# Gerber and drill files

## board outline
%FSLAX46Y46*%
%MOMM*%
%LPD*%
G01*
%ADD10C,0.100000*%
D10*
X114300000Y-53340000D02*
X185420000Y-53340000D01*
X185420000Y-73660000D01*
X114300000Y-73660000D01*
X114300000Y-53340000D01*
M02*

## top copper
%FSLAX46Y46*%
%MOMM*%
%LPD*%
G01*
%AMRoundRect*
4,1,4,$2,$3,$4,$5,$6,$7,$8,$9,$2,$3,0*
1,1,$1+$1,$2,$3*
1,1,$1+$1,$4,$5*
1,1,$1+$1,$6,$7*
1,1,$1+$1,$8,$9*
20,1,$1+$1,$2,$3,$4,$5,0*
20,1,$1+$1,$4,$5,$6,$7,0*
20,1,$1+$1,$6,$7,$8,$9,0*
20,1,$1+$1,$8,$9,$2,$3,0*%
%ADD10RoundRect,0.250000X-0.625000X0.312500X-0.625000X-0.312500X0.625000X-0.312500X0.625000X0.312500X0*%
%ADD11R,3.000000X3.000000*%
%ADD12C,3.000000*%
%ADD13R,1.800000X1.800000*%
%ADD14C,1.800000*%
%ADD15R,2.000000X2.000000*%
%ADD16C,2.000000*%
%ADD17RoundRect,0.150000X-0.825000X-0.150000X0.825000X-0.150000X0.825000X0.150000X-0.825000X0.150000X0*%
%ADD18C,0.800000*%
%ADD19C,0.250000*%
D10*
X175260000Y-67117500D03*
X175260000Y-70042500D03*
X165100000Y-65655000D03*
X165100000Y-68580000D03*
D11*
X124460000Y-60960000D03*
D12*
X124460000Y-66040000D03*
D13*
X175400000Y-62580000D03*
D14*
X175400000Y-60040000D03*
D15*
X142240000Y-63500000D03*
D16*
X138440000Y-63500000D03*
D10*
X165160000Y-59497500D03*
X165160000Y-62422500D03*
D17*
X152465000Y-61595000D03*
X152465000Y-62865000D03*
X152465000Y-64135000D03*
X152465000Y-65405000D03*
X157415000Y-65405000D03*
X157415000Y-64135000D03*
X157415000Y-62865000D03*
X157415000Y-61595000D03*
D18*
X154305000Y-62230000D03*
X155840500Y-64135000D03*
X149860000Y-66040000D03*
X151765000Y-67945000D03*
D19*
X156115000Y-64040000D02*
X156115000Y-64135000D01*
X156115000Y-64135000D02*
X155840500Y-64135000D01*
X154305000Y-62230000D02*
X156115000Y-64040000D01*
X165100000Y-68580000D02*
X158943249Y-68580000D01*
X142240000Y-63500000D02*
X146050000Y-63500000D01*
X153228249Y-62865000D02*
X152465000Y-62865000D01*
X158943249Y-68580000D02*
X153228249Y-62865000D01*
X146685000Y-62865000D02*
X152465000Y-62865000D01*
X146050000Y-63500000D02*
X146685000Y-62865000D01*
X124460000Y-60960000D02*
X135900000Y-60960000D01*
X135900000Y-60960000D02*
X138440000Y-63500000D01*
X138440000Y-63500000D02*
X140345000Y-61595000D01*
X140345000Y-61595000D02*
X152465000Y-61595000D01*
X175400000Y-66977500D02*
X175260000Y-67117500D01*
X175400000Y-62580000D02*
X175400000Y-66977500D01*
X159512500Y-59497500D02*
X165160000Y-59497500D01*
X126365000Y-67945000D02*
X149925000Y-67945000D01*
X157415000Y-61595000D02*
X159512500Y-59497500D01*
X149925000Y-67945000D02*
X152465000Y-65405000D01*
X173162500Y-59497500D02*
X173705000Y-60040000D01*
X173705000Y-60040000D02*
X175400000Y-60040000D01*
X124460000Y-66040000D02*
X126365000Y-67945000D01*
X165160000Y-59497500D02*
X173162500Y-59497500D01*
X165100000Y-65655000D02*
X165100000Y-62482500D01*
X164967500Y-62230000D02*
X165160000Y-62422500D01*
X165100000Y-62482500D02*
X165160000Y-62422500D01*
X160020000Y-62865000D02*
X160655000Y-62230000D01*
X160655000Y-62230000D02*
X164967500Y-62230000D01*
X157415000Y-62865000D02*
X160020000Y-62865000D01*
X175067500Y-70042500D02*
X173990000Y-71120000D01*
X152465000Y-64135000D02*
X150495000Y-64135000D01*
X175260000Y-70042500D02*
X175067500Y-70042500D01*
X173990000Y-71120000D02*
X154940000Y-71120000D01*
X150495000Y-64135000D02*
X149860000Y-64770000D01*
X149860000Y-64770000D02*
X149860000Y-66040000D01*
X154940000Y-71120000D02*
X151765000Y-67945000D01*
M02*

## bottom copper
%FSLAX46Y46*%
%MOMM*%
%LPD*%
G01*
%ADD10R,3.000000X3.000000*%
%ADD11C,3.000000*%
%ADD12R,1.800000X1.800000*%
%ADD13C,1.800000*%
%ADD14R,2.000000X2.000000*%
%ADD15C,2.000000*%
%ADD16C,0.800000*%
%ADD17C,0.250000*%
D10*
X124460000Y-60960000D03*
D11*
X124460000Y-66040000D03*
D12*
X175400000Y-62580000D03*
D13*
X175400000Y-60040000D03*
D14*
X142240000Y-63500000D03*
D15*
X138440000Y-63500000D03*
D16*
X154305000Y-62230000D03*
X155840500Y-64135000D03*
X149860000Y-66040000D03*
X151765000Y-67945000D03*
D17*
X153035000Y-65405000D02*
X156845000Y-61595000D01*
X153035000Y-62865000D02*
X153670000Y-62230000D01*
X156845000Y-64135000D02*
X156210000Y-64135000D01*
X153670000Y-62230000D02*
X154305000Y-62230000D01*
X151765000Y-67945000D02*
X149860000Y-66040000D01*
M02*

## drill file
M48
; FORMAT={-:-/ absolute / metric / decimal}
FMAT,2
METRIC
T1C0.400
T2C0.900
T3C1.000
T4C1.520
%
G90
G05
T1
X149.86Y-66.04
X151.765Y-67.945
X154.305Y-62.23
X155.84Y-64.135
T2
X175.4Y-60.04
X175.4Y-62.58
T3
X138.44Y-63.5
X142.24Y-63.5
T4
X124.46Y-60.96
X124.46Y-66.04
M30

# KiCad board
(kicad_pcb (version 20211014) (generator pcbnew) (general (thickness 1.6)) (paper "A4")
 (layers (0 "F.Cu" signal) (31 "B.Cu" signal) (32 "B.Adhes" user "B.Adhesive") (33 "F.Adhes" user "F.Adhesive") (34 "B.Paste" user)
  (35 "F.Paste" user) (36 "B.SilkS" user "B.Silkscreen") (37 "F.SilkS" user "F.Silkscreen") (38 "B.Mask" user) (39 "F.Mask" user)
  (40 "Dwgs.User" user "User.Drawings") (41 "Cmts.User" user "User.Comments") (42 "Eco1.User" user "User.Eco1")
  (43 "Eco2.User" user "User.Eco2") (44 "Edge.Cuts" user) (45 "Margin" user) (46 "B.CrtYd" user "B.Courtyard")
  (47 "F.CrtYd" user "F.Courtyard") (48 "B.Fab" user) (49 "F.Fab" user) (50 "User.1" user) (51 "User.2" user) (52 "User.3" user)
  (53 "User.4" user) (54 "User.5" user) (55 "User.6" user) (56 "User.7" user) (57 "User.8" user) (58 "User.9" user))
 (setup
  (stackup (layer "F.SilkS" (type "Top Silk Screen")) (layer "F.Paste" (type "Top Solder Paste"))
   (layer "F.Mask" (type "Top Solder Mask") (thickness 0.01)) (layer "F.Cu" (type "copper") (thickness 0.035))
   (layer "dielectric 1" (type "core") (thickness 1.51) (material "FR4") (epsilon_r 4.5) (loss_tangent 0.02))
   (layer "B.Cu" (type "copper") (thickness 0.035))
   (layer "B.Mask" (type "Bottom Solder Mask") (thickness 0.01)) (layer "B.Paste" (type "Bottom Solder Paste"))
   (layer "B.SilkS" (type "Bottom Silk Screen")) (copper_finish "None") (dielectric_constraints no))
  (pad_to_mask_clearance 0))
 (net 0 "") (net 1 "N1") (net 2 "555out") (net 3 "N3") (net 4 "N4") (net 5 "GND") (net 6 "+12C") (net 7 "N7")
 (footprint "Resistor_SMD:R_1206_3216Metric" (layer "F.Cu") (at 175.26 68.58 -90)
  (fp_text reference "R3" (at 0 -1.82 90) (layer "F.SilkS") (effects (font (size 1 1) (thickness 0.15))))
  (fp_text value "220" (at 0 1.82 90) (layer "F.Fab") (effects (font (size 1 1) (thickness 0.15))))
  (pad "1" smd roundrect (at -1.4625 0 270) (size 1.125 1.75) (layers "F.Cu" "F.Paste" "F.Mask") (roundrect_rratio 0.222222) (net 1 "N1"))
  (pad "2" smd roundrect (at 1.4625 0 270) (size 1.125 1.75) (layers "F.Cu" "F.Paste" "F.Mask") (roundrect_rratio 0.222222) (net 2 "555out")))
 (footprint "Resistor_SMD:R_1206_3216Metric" (layer "F.Cu") (at 165.1 67.1175 -90)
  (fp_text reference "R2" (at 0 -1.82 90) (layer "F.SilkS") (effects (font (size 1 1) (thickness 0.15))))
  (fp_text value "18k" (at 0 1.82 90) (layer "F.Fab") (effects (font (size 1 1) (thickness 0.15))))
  (pad "1" smd roundrect (at -1.4625 0 270) (size 1.125 1.75) (layers "F.Cu" "F.Paste" "F.Mask") (roundrect_rratio 0.222222) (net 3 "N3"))
  (pad "2" smd roundrect (at 1.4625 0 270) (size 1.125 1.75) (layers "F.Cu" "F.Paste" "F.Mask") (roundrect_rratio 0.222222) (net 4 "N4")))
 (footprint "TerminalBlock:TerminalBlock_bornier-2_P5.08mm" (layer "F.Cu") (at 124.46 60.96 -90)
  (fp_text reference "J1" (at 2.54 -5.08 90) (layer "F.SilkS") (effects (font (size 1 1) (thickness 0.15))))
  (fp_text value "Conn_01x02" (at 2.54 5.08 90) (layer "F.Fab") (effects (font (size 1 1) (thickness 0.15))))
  (pad "1" thru_hole rect (at 0 0 270) (size 3 3) (drill 1.52) (layers *.Cu *.Mask) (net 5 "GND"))
  (pad "2" thru_hole circle (at 5.08 0 270) (size 3 3) (drill 1.52) (layers *.Cu *.Mask) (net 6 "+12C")))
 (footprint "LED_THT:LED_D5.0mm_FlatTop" (layer "F.Cu") (at 175.4 62.58 90)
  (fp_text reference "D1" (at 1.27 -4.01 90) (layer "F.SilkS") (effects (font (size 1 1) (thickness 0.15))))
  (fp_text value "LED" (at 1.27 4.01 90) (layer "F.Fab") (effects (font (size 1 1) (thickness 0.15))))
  (pad "1" thru_hole rect (at 0 0 90) (size 1.8 1.8) (drill 0.9) (layers *.Cu *.Mask) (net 1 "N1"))
  (pad "2" thru_hole circle (at 2.54 0 90) (size 1.8 1.8) (drill 0.9) (layers *.Cu *.Mask) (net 6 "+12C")))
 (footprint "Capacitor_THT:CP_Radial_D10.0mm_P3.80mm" (layer "F.Cu") (at 142.24 63.5 180)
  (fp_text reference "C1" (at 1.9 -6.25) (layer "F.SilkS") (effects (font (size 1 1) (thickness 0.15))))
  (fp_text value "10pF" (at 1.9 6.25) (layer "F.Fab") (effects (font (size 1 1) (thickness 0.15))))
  (pad "1" thru_hole rect (at 0 0 180) (size 2 2) (drill 1) (layers *.Cu *.Mask) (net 4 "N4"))
  (pad "2" thru_hole circle (at 3.8 0 180) (size 2 2) (drill 1) (layers *.Cu *.Mask) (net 5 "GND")))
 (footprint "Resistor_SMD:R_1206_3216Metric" (layer "F.Cu") (at 165.16 60.96 -90)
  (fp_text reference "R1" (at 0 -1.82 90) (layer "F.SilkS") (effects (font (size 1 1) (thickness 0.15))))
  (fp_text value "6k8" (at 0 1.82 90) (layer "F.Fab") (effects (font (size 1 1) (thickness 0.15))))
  (pad "1" smd roundrect (at -1.4625 0 270) (size 1.125 1.75) (layers "F.Cu" "F.Paste" "F.Mask") (roundrect_rratio 0.222222) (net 6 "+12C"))
  (pad "2" smd roundrect (at 1.4625 0 270) (size 1.125 1.75) (layers "F.Cu" "F.Paste" "F.Mask") (roundrect_rratio 0.222222) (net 3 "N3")))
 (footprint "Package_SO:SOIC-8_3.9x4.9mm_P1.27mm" (layer "F.Cu") (at 154.94 63.5)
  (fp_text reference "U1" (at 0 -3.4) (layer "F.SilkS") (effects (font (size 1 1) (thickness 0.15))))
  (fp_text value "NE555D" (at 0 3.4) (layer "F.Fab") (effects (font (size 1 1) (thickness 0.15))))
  (pad "1" smd roundrect (at -2.475 -1.905) (size 1.95 0.6) (layers "F.Cu" "F.Paste" "F.Mask") (roundrect_rratio 0.25) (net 5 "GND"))
  (pad "2" smd roundrect (at -2.475 -0.635) (size 1.95 0.6) (layers "F.Cu" "F.Paste" "F.Mask") (roundrect_rratio 0.25) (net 4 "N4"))
  (pad "3" smd roundrect (at -2.475 0.635) (size 1.95 0.6) (layers "F.Cu" "F.Paste" "F.Mask") (roundrect_rratio 0.25) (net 2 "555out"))
  (pad "4" smd roundrect (at -2.475 1.905) (size 1.95 0.6) (layers "F.Cu" "F.Paste" "F.Mask") (roundrect_rratio 0.25) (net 6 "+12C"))
  (pad "5" smd roundrect (at 2.475 1.905) (size 1.95 0.6) (layers "F.Cu" "F.Paste" "F.Mask") (roundrect_rratio 0.25) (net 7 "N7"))
  (pad "6" smd roundrect (at 2.475 0.635) (size 1.95 0.6) (layers "F.Cu" "F.Paste" "F.Mask") (roundrect_rratio 0.25) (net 4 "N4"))
  (pad "7" smd roundrect (at 2.475 -0.635) (size 1.95 0.6) (layers "F.Cu" "F.Paste" "F.Mask") (roundrect_rratio 0.25) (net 3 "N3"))
  (pad "8" smd roundrect (at 2.475 -1.905) (size 1.95 0.6) (layers "F.Cu" "F.Paste" "F.Mask") (roundrect_rratio 0.25) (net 6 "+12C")))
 (gr_rect (start 114.3 53.34) (end 185.42 73.66) (layer "Edge.Cuts") (width 0.1) (fill none))
 (segment (start 156.115 64.04) (end 156.115 64.135) (width 0.25) (layer "F.Cu") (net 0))
 (segment (start 156.115 64.135) (end 155.8405 64.135) (width 0.25) (layer "F.Cu") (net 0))
 (segment (start 154.305 62.23) (end 156.115 64.04) (width 0.25) (layer "F.Cu") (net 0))
 (via (at 154.305 62.23) (size 0.8) (drill 0.4) (layers "F.Cu" "B.Cu") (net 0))
 (via (at 155.8405 64.135) (size 0.8) (drill 0.4) (layers "F.Cu" "B.Cu") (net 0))
 (segment (start 153.035 65.405) (end 156.845 61.595) (width 0.25) (layer "B.Cu") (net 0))
 (segment (start 153.035 62.865) (end 153.67 62.23) (width 0.25) (layer "B.Cu") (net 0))
 (segment (start 156.845 64.135) (end 156.21 64.135) (width 0.25) (layer "B.Cu") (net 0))
 (segment (start 153.67 62.23) (end 154.305 62.23) (width 0.25) (layer "B.Cu") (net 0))
 (segment (start 165.1 68.58) (end 158.943249 68.58) (width 0.25) (layer "F.Cu") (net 4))
 (segment (start 142.24 63.5) (end 146.05 63.5) (width 0.25) (layer "F.Cu") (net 4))
 (segment (start 153.228249 62.865) (end 152.465 62.865) (width 0.25) (layer "F.Cu") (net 4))
 (segment (start 158.943249 68.58) (end 153.228249 62.865) (width 0.25) (layer "F.Cu") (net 4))
 (segment (start 146.685 62.865) (end 152.465 62.865) (width 0.25) (layer "F.Cu") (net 4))
 (segment (start 146.05 63.5) (end 146.685 62.865) (width 0.25) (layer "F.Cu") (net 4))
 (segment (start 124.46 60.96) (end 135.9 60.96) (width 0.25) (layer "F.Cu") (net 5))
 (segment (start 135.9 60.96) (end 138.44 63.5) (width 0.25) (layer "F.Cu") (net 5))
 (segment (start 138.44 63.5) (end 140.345 61.595) (width 0.25) (layer "F.Cu") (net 5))
 (segment (start 140.345 61.595) (end 152.465 61.595) (width 0.25) (layer "F.Cu") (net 5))
 (segment (start 175.4 66.9775) (end 175.26 67.1175) (width 0.25) (layer "F.Cu") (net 1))
 (segment (start 175.4 62.58) (end 175.4 66.9775) (width 0.25) (layer "F.Cu") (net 1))
 (segment (start 159.5125 59.4975) (end 165.16 59.4975) (width 0.25) (layer "F.Cu") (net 6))
 (segment (start 126.365 67.945) (end 149.925 67.945) (width 0.25) (layer "F.Cu") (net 6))
 (segment (start 157.415 61.595) (end 159.5125 59.4975) (width 0.25) (layer "F.Cu") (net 6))
 (segment (start 149.925 67.945) (end 152.465 65.405) (width 0.25) (layer "F.Cu") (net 6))
 (segment (start 173.1625 59.4975) (end 173.705 60.04) (width 0.25) (layer "F.Cu") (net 6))
 (segment (start 173.705 60.04) (end 175.4 60.04) (width 0.25) (layer "F.Cu") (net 6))
 (segment (start 124.46 66.04) (end 126.365 67.945) (width 0.25) (layer "F.Cu") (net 6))
 (segment (start 165.16 59.4975) (end 173.1625 59.4975) (width 0.25) (layer "F.Cu") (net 6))
 (segment (start 165.1 65.655) (end 165.1 62.4825) (width 0.25) (layer "F.Cu") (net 3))
 (segment (start 164.9675 62.23) (end 165.16 62.4225) (width 0.25) (layer "F.Cu") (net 3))
 (segment (start 165.1 62.4825) (end 165.16 62.4225) (width 0.25) (layer "F.Cu") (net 3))
 (segment (start 160.02 62.865) (end 160.655 62.23) (width 0.25) (layer "F.Cu") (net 3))
 (segment (start 160.655 62.23) (end 164.9675 62.23) (width 0.25) (layer "F.Cu") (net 3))
 (segment (start 157.415 62.865) (end 160.02 62.865) (width 0.25) (layer "F.Cu") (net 3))
 (segment (start 175.0675 70.0425) (end 173.99 71.12) (width 0.25) (layer "F.Cu") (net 2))
 (segment (start 152.465 64.135) (end 150.495 64.135) (width 0.25) (layer "F.Cu") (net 2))
 (segment (start 175.26 70.0425) (end 175.0675 70.0425) (width 0.25) (layer "F.Cu") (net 2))
 (segment (start 173.99 71.12) (end 154.94 71.12) (width 0.25) (layer "F.Cu") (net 2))
 (segment (start 150.495 64.135) (end 149.86 64.77) (width 0.25) (layer "F.Cu") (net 2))
 (segment (start 149.86 64.77) (end 149.86 66.04) (width 0.25) (layer "F.Cu") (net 2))
 (segment (start 154.94 71.12) (end 151.765 67.945) (width 0.25) (layer "F.Cu") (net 2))
 (via (at 149.86 66.04) (size 0.8) (drill 0.4) (layers "F.Cu" "B.Cu") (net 2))
 (via (at 151.765 67.945) (size 0.8) (drill 0.4) (layers "F.Cu" "B.Cu") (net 2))
 (segment (start 151.765 67.945) (end 149.86 66.04) (width 0.25) (layer "B.Cu") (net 2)))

